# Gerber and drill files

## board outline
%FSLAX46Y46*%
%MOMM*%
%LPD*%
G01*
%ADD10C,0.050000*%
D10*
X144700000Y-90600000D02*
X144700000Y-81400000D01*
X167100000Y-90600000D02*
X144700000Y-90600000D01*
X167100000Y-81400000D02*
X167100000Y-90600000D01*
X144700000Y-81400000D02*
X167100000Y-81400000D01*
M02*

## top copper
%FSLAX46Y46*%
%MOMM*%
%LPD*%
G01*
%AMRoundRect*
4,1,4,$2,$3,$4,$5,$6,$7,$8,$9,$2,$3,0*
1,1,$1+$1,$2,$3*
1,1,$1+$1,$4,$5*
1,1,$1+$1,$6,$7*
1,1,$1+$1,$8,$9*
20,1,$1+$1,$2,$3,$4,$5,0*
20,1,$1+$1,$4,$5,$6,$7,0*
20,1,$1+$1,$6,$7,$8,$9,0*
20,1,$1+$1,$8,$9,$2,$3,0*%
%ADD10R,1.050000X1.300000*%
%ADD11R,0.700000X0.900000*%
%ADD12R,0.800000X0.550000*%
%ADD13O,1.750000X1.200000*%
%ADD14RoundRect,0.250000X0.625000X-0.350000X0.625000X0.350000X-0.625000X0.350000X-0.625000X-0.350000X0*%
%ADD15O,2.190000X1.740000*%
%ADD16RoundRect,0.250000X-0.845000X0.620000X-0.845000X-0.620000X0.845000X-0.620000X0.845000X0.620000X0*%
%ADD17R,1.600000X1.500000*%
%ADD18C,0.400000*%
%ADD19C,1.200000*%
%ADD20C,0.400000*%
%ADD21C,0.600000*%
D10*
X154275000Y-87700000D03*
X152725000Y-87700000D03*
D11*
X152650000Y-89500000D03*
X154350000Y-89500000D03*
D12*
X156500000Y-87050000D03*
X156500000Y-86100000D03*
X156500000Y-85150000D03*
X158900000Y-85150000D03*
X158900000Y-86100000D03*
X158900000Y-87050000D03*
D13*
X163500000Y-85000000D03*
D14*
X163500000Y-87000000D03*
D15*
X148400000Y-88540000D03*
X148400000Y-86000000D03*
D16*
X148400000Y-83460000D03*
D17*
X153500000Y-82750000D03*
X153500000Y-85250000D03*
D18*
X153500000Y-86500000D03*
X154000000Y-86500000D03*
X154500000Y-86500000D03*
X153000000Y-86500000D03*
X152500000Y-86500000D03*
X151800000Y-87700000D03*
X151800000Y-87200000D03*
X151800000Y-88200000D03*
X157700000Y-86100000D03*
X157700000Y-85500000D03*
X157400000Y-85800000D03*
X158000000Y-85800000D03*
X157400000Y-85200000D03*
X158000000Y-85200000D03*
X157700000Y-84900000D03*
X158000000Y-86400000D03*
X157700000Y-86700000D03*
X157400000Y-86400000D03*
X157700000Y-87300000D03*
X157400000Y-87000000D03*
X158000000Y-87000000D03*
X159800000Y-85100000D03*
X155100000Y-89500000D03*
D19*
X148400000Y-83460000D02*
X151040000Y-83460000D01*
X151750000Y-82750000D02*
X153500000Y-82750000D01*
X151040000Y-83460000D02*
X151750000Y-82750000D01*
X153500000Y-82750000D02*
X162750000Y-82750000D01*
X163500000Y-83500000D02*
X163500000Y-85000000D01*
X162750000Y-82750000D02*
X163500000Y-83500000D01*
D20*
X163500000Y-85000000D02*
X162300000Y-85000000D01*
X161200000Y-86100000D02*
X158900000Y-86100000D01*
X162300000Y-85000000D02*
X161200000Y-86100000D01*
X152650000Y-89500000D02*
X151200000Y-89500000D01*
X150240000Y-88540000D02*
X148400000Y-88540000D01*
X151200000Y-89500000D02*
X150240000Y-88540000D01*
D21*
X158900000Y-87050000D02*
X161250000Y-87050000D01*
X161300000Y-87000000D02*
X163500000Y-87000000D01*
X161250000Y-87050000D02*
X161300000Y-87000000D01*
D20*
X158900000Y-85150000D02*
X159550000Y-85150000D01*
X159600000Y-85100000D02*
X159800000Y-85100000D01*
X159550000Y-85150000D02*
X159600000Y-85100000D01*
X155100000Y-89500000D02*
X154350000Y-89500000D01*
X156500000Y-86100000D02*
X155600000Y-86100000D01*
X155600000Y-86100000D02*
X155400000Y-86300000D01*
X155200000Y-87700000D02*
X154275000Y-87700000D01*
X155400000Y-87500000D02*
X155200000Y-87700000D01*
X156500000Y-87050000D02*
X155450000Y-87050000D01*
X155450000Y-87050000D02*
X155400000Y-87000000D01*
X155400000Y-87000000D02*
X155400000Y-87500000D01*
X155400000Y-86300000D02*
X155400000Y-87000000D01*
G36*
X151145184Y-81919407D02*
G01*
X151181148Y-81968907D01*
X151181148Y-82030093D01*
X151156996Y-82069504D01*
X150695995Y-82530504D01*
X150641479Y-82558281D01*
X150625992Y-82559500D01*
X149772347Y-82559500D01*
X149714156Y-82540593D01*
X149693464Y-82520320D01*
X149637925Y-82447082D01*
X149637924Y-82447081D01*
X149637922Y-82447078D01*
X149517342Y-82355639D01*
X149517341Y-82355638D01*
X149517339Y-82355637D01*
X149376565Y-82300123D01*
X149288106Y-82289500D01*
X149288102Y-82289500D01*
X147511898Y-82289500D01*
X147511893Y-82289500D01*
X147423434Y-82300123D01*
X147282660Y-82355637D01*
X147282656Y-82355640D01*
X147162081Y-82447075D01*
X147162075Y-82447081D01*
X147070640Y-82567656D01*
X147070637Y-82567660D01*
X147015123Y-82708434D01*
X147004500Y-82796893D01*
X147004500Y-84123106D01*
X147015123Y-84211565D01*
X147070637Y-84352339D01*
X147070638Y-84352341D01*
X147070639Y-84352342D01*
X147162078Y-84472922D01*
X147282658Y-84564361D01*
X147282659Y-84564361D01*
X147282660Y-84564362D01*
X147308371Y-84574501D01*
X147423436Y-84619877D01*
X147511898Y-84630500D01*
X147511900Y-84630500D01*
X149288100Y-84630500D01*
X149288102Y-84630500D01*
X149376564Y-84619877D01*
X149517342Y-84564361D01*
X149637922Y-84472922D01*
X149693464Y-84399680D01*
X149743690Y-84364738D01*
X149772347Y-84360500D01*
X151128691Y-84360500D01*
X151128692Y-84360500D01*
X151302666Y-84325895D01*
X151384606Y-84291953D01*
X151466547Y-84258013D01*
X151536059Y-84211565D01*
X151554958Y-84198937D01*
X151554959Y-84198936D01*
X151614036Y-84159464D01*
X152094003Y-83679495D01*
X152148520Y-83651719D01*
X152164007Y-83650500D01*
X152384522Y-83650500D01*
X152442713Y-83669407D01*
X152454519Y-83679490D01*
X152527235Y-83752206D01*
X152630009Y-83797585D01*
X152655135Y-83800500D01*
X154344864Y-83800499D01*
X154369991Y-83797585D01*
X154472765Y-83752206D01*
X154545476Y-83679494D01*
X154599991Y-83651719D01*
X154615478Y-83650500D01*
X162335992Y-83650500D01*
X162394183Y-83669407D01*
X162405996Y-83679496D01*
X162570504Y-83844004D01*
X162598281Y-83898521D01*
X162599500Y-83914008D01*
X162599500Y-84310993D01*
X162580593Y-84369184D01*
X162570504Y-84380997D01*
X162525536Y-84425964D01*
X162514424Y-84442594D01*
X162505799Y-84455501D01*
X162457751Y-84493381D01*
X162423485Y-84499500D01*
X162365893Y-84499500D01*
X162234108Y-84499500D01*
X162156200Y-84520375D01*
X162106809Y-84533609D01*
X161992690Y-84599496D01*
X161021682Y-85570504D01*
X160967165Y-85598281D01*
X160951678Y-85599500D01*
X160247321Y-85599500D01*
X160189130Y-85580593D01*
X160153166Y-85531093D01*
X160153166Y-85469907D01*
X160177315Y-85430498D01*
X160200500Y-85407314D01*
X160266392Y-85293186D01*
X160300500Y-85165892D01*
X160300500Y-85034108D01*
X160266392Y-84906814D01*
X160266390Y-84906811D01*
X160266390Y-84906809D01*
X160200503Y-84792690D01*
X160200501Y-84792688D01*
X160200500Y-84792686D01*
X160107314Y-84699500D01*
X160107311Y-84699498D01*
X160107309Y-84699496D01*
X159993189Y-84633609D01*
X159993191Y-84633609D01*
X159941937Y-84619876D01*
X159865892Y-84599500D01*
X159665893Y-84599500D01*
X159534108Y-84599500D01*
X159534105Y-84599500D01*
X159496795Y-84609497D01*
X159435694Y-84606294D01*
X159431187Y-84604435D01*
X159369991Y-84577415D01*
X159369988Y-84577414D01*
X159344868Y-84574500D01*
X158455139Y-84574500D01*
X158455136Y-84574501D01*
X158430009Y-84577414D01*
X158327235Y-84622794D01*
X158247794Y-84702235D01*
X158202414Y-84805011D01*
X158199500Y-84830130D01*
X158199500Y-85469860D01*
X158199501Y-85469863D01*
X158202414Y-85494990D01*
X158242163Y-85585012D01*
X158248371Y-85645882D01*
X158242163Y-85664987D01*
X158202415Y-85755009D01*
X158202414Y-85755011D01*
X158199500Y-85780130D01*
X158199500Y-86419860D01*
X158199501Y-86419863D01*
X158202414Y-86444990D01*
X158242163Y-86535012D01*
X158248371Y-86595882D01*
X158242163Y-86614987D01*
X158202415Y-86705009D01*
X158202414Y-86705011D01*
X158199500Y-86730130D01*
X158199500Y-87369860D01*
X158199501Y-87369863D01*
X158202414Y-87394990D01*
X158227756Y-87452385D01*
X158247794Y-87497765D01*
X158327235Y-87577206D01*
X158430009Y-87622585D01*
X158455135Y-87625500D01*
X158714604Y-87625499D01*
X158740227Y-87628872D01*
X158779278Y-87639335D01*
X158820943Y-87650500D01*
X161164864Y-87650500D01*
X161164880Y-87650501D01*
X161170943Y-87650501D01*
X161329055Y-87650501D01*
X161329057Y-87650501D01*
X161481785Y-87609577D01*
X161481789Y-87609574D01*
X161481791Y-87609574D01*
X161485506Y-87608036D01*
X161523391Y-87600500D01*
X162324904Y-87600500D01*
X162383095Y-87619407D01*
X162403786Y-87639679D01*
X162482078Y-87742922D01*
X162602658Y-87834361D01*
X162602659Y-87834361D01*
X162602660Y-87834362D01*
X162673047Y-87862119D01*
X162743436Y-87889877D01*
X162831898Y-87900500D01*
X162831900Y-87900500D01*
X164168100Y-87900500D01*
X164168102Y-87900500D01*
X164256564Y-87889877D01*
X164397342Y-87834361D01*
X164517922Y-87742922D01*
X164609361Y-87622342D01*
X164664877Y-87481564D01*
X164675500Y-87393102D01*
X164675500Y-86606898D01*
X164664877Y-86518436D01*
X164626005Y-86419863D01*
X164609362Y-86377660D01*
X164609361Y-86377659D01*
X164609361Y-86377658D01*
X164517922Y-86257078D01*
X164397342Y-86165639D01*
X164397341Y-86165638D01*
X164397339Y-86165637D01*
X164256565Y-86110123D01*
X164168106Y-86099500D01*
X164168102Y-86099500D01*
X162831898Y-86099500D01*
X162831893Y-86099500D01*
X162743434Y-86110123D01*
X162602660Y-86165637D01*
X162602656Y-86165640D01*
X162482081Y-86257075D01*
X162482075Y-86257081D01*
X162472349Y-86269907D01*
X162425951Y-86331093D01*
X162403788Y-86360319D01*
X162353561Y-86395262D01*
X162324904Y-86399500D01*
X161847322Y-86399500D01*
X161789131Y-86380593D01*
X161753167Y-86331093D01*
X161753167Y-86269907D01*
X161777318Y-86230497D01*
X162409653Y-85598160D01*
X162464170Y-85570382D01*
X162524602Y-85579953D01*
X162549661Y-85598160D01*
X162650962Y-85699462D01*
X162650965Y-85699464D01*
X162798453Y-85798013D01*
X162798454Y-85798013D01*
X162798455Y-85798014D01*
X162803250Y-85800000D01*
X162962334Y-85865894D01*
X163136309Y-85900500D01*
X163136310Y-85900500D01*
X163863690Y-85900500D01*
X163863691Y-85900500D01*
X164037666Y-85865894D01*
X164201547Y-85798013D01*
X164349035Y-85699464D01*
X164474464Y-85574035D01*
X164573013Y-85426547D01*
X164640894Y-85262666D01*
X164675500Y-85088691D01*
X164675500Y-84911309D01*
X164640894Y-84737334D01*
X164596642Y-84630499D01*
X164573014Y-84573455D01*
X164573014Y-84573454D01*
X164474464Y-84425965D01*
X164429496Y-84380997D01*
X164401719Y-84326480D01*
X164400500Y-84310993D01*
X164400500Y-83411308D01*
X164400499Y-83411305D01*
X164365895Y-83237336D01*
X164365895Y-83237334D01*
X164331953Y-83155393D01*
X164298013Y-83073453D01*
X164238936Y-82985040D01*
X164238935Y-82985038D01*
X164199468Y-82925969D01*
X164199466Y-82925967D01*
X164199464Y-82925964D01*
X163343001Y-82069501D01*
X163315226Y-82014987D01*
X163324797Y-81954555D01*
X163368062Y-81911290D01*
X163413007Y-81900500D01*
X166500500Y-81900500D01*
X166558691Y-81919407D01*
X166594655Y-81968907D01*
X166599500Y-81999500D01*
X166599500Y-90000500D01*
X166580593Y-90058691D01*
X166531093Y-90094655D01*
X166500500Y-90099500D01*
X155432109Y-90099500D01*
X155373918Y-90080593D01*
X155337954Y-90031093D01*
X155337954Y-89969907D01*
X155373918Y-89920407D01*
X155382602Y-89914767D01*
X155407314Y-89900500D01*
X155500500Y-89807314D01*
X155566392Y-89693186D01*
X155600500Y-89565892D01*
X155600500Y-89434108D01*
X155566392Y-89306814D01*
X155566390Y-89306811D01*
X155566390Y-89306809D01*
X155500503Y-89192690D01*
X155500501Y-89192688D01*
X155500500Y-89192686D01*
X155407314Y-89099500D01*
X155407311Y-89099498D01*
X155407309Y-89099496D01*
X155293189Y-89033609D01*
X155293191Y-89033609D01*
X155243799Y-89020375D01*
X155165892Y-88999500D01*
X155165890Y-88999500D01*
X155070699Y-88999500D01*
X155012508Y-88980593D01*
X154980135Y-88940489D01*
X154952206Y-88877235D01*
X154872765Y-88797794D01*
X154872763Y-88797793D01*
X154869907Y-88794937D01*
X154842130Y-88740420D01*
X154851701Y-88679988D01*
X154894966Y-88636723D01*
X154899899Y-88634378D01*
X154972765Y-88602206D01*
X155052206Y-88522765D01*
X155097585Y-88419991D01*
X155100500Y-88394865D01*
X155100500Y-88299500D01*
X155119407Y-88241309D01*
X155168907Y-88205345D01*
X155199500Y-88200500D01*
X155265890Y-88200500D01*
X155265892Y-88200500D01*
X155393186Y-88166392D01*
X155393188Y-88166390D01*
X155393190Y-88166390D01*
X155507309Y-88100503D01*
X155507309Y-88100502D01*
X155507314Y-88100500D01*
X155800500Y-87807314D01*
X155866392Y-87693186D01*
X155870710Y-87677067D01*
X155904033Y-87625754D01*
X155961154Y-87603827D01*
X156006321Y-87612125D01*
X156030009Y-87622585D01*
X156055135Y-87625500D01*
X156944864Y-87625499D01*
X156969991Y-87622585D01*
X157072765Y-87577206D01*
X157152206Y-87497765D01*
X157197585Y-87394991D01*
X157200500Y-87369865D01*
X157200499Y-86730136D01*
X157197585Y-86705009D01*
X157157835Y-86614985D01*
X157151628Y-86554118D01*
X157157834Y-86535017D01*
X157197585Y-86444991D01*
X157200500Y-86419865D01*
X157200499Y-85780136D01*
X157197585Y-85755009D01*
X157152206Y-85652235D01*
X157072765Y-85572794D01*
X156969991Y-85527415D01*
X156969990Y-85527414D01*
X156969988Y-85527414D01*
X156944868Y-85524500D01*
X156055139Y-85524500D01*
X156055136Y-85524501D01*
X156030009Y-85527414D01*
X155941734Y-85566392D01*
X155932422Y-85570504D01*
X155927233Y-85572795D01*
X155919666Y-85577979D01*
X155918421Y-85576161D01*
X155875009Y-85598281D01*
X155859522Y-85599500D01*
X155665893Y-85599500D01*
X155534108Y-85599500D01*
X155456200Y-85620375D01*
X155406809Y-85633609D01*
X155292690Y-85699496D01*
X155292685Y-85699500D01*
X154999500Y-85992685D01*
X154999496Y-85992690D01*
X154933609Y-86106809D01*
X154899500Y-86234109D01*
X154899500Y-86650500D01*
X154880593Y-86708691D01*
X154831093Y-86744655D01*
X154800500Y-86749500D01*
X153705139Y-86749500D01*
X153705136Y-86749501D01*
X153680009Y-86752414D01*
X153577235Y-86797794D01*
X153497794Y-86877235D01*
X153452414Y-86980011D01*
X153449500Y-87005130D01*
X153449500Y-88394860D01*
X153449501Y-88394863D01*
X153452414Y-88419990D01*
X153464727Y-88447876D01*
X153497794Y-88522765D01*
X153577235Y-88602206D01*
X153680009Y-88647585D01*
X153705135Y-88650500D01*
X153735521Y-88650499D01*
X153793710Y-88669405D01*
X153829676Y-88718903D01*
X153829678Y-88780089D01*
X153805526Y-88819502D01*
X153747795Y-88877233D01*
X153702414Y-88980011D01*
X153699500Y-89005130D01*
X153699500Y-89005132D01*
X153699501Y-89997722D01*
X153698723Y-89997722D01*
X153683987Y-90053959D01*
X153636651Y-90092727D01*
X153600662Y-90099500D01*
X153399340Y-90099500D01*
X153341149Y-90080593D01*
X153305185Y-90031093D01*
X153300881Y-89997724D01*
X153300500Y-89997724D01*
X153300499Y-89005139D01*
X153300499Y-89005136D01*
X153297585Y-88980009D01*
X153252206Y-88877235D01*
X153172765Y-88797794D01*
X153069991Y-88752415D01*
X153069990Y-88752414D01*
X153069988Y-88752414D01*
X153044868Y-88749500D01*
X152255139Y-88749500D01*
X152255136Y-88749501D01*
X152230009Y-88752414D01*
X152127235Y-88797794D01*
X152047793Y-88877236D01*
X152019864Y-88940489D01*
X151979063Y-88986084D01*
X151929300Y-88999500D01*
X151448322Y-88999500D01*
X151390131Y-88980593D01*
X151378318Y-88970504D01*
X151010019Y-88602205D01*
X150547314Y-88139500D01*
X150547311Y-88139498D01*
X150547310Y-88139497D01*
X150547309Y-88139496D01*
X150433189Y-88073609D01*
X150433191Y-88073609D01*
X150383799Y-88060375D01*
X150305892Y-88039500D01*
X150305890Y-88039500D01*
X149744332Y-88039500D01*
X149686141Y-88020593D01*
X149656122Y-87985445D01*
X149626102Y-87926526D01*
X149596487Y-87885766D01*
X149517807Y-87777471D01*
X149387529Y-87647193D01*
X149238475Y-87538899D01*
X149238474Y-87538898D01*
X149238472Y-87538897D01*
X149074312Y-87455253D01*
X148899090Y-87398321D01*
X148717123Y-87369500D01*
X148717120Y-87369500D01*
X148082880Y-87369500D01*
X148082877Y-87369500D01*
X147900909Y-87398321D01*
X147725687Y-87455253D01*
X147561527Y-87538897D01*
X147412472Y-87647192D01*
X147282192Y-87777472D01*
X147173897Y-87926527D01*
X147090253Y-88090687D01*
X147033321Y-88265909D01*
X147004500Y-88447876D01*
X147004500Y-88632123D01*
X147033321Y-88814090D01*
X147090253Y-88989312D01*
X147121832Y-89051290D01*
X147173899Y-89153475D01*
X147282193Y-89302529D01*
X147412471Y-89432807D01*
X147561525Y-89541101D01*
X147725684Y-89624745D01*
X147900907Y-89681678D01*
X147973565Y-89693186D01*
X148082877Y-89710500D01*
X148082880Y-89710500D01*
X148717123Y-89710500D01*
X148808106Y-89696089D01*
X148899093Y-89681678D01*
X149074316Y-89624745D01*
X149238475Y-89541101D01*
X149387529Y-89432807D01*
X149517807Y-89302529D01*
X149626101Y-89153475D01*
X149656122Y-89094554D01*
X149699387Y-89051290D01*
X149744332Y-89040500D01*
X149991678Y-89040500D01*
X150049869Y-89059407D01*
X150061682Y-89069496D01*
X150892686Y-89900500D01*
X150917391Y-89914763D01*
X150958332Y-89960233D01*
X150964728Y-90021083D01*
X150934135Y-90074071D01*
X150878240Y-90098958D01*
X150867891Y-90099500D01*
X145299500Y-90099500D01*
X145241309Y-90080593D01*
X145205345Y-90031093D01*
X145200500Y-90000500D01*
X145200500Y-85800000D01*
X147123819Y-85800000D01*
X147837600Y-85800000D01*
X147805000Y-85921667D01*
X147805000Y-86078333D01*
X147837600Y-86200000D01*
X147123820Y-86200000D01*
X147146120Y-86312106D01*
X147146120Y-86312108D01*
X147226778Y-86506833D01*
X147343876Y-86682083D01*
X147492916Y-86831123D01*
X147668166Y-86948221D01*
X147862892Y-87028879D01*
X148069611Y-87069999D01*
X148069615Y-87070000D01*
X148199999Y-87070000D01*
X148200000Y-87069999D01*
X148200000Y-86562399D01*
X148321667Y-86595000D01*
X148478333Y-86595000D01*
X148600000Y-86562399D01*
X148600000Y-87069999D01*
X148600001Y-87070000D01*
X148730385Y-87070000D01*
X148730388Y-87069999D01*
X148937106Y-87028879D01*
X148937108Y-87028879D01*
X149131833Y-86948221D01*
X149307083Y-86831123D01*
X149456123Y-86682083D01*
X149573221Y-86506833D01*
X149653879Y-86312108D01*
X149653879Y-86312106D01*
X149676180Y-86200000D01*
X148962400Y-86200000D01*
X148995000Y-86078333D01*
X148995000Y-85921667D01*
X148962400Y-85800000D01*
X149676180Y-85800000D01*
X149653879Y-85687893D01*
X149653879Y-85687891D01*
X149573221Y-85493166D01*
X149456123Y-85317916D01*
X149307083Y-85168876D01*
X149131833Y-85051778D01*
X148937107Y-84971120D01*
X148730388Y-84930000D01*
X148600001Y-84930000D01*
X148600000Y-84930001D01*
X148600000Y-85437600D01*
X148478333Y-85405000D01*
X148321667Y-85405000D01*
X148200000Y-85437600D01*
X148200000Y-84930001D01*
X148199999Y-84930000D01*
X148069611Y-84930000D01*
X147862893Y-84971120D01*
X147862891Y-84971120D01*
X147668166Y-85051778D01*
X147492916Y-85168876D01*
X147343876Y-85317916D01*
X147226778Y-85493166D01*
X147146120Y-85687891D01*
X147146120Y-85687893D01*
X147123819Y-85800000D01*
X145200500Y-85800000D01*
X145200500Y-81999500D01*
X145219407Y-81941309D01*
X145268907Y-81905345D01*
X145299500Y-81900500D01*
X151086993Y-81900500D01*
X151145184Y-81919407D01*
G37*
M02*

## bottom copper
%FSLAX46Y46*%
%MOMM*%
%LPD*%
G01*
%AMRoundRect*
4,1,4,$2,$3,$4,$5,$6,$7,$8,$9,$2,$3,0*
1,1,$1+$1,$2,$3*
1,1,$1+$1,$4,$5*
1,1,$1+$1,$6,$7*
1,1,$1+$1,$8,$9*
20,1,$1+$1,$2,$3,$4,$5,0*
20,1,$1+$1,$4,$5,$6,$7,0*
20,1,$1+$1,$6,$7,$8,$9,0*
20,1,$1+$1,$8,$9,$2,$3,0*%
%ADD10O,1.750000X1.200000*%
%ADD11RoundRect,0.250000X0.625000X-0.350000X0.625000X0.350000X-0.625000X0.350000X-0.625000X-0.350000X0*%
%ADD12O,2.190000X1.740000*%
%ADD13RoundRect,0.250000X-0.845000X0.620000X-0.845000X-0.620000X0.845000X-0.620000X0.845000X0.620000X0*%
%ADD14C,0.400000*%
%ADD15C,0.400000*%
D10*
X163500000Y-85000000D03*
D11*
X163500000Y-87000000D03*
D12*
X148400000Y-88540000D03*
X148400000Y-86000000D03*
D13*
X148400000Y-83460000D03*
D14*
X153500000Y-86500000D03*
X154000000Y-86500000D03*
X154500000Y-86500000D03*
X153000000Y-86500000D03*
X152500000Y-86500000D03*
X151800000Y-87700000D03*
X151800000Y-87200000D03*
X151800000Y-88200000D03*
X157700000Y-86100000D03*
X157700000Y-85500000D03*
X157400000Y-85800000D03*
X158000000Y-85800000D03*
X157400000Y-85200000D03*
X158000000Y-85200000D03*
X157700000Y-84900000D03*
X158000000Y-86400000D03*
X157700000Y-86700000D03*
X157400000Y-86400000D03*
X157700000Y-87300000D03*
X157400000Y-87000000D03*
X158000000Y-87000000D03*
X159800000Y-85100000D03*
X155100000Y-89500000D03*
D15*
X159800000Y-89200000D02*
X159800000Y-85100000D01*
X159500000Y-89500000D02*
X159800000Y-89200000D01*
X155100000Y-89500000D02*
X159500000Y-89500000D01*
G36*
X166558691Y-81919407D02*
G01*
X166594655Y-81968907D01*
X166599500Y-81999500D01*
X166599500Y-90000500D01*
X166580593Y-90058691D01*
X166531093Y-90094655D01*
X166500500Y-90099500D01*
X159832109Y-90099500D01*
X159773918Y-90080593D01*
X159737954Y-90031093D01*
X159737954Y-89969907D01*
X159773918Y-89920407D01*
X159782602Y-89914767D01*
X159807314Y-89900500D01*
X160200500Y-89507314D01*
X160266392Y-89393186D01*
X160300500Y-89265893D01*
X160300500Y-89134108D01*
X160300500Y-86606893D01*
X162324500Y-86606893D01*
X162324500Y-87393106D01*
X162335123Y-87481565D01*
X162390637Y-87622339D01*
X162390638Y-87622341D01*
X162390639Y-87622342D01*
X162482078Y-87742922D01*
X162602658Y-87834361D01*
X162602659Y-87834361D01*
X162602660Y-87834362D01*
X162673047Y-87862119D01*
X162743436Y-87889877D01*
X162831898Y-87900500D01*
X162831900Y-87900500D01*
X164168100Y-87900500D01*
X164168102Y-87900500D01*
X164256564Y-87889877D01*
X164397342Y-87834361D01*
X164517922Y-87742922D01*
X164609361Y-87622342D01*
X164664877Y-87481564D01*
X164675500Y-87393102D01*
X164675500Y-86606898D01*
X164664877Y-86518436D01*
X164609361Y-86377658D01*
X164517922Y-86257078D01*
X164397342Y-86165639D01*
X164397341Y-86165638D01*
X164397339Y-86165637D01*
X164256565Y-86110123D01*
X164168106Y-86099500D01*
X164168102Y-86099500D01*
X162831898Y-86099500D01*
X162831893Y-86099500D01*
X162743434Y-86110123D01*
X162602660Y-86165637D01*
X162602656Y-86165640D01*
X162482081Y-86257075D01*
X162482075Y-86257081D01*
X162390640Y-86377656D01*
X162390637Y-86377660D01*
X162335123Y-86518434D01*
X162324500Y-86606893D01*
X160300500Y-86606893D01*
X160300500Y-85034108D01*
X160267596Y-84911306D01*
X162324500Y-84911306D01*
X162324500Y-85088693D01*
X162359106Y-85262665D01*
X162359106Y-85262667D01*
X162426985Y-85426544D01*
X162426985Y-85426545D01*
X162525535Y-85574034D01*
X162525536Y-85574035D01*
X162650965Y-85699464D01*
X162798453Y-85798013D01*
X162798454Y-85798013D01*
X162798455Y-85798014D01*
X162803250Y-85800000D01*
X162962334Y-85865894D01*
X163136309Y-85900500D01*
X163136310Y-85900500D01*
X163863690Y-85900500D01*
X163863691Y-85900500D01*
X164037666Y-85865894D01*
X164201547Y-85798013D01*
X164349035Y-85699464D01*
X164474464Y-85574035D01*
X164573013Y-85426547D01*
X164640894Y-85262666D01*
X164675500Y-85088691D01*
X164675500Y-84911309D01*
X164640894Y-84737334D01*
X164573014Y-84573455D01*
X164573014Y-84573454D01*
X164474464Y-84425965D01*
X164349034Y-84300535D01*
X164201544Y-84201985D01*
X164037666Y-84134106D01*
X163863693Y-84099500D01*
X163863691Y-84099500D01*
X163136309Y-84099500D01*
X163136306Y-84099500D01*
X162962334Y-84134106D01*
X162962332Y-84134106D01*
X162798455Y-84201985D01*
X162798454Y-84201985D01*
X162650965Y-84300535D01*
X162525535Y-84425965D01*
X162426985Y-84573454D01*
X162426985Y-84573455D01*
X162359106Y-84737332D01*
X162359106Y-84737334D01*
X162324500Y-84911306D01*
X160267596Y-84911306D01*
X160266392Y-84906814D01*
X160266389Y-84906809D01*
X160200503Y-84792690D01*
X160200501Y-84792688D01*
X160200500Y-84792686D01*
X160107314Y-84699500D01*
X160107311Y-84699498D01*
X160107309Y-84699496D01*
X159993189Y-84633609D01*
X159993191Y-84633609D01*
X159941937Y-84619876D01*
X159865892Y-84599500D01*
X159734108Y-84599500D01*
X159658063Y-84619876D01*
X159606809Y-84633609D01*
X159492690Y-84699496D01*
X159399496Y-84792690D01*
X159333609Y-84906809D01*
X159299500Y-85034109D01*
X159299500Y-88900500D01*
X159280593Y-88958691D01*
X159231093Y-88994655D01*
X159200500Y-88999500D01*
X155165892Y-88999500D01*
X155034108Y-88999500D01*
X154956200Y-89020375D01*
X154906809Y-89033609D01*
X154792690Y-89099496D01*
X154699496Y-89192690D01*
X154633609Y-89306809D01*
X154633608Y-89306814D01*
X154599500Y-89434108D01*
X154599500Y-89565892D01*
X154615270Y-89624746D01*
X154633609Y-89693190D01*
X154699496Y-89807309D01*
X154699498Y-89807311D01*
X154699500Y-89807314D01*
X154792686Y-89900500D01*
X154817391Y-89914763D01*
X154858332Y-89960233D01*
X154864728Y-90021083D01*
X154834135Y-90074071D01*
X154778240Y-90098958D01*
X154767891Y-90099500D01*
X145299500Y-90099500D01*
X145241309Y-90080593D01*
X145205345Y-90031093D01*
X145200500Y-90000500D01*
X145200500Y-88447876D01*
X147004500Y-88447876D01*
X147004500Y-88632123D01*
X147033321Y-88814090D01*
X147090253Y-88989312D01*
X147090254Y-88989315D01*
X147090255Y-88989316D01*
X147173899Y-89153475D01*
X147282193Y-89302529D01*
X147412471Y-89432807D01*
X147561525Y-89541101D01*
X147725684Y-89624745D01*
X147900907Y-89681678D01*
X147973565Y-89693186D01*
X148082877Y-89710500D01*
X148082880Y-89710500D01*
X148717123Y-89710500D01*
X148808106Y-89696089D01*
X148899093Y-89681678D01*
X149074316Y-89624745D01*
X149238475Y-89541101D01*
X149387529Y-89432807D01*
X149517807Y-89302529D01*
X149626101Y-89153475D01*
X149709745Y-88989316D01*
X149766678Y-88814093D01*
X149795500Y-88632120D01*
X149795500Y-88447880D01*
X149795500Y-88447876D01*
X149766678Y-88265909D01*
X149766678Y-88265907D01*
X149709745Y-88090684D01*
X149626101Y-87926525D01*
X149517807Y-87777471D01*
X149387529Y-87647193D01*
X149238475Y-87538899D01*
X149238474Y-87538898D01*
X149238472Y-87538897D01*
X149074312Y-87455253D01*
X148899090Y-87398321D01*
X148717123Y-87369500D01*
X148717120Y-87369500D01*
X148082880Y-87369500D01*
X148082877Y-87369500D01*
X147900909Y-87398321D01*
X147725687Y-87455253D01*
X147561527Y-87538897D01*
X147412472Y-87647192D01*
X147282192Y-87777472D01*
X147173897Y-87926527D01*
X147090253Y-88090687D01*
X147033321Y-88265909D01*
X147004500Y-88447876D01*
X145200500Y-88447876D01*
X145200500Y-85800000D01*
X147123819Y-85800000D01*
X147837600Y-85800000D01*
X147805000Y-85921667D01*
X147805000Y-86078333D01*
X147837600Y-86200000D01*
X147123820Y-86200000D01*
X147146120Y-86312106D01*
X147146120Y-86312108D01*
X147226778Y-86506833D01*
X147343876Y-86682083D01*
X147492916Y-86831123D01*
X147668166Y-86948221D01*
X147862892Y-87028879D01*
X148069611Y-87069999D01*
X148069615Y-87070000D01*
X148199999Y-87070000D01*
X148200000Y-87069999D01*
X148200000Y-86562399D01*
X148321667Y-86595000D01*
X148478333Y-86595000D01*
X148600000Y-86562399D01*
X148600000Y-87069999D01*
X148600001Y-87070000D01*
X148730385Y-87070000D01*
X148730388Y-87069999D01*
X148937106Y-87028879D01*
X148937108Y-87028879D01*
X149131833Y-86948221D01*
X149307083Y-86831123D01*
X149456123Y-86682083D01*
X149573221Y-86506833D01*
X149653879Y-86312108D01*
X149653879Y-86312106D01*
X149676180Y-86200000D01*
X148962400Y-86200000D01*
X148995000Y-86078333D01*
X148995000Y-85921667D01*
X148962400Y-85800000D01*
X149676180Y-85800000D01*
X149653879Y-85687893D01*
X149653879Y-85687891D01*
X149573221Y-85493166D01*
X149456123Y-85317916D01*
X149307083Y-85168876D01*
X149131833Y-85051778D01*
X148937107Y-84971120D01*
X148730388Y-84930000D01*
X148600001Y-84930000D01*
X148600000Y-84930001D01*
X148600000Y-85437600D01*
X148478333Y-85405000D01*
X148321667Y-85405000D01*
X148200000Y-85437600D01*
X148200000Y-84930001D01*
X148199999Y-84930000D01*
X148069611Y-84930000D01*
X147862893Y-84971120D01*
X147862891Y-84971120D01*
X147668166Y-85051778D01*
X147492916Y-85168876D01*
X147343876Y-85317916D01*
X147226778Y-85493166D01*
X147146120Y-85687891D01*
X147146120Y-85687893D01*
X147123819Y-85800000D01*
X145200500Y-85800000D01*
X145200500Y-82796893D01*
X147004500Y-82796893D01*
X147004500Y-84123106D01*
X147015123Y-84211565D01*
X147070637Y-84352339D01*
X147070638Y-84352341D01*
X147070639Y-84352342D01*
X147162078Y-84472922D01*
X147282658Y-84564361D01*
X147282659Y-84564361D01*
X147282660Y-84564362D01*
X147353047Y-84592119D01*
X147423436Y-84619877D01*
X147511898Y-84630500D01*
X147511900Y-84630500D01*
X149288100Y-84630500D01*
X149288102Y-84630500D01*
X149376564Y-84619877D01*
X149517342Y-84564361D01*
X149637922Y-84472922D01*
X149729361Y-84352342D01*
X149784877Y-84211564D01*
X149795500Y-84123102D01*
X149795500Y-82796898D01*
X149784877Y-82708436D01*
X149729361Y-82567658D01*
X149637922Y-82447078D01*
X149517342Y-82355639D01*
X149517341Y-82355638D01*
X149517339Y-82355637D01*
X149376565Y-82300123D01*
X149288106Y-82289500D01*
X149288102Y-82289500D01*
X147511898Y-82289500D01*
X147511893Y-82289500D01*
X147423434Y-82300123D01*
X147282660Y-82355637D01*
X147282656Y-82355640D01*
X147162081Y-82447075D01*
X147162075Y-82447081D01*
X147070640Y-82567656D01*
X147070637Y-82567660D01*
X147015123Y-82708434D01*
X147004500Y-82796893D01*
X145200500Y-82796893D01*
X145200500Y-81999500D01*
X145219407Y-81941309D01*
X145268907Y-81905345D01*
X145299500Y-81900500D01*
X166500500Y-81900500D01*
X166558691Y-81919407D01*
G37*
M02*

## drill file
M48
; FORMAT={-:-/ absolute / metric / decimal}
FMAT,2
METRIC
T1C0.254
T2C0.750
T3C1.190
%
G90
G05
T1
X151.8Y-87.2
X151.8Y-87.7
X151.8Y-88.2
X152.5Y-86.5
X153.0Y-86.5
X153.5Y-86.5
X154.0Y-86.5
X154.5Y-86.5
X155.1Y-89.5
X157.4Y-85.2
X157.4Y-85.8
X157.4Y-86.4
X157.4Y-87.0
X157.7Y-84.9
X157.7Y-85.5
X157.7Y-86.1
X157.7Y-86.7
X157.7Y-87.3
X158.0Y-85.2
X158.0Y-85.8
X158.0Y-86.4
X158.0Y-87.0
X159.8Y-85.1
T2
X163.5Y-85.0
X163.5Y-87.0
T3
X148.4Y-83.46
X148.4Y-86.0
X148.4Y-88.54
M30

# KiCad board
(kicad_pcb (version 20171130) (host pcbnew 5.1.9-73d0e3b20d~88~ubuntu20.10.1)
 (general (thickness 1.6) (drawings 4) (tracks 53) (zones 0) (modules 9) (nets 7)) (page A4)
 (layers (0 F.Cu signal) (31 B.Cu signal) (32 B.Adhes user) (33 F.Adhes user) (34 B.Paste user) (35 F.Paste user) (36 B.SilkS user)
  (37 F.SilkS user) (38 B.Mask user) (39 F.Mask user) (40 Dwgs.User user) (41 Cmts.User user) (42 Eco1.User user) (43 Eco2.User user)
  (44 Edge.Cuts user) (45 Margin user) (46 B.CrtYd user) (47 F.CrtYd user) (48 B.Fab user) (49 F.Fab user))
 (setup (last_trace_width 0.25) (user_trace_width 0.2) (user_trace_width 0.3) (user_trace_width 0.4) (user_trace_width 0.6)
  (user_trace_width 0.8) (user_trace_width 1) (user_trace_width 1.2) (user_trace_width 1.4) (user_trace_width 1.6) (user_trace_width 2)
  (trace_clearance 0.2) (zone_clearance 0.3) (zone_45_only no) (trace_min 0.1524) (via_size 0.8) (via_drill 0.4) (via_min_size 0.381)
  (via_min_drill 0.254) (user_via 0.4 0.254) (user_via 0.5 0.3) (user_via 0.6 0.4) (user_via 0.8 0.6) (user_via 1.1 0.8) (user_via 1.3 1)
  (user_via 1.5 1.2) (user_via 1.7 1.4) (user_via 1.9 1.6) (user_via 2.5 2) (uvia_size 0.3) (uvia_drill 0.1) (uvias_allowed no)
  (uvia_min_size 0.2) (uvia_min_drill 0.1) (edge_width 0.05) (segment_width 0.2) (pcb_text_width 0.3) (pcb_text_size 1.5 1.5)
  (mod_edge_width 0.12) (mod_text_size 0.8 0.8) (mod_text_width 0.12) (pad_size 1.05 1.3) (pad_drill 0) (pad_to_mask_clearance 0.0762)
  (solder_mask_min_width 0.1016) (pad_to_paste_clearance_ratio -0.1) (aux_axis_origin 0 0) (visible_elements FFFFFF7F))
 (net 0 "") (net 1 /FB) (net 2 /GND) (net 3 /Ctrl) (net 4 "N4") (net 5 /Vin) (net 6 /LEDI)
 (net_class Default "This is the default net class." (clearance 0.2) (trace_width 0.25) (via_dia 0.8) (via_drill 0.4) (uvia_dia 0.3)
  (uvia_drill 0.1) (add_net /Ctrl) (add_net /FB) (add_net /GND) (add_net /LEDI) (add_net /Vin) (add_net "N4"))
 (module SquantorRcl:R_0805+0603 (layer F.Cu) (at 153.5 87.7)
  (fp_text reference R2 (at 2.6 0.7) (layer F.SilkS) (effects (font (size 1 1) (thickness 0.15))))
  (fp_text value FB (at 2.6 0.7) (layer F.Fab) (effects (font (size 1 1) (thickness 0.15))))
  (pad 2 smd rect (at 0.775 0) (size 1.05 1.3) (layers F.Cu F.Paste F.Mask) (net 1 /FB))
  (pad 1 smd rect (at -0.775 0) (size 1.05 1.3) (layers F.Cu F.Paste F.Mask) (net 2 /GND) (zone_connect 2)))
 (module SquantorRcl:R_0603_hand (layer F.Cu) (at 153.5 89.5 180)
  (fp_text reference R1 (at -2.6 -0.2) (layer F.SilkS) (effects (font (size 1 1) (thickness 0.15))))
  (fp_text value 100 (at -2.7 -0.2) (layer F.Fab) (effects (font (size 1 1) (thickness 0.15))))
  (pad 2 smd rect (at 0.85 0 180) (size 0.7 0.9) (layers F.Cu F.Paste F.Mask) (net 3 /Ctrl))
  (pad 1 smd rect (at -0.85 0 180) (size 0.7 0.9) (layers F.Cu F.Paste F.Mask) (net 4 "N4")))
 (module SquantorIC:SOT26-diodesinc (layer F.Cu) (at 157.7 86.1 90)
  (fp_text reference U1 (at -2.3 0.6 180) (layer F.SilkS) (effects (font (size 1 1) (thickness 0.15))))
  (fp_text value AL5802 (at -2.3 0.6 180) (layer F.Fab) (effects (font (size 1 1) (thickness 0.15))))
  (pad 6 smd rect (at -0.95 -1.2 90) (size 0.55 0.8) (layers F.Cu F.Paste F.Mask) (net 1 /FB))
  (pad 5 smd rect (at 0 -1.2 90) (size 0.55 0.8) (layers F.Cu F.Paste F.Mask) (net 1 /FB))
  (pad 4 smd rect (at 0.95 -1.2 90) (size 0.55 0.8) (layers F.Cu F.Paste F.Mask) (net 2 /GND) (zone_connect 2))
  (pad 3 smd rect (at 0.95 1.2 90) (size 0.55 0.8) (layers F.Cu F.Paste F.Mask) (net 4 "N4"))
  (pad 2 smd rect (at 0 1.2 90) (size 0.55 0.8) (layers F.Cu F.Paste F.Mask) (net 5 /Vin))
  (pad 1 smd rect (at -0.95 1.2 90) (size 0.55 0.8) (layers F.Cu F.Paste F.Mask) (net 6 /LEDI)))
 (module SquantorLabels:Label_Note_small (layer F.Cu) (at 156 82.9)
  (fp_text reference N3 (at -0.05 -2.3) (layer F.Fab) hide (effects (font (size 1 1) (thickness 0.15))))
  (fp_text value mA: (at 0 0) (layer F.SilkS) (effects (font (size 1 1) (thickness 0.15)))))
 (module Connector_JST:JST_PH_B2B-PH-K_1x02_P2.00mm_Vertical (layer F.Cu) (at 163.5 87 90)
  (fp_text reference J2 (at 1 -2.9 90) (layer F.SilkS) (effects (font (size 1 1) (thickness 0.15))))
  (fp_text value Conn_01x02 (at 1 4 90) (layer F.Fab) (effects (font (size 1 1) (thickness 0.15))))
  (pad 2 thru_hole oval (at 2 0 90) (size 1.2 1.75) (drill 0.75) (layers *.Cu *.Mask) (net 5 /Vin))
  (pad 1 thru_hole roundrect (at 0 0 90) (size 1.2 1.75) (drill 0.75) (layers *.Cu *.Mask) (roundrect_rratio 0.208333) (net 6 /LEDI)))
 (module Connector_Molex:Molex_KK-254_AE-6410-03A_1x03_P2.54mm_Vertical (layer F.Cu) (at 148.4 83.46 270)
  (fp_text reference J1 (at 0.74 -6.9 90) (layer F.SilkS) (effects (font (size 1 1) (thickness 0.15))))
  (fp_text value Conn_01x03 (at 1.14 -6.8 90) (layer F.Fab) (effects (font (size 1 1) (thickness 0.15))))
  (pad 3 thru_hole oval (at 5.08 0 270) (size 1.74 2.19) (drill 1.19) (layers *.Cu *.Mask) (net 3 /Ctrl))
  (pad 2 thru_hole oval (at 2.54 0 270) (size 1.74 2.19) (drill 1.19) (layers *.Cu *.Mask) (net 2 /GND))
  (pad 1 thru_hole roundrect (at 0 0 270) (size 1.74 2.19) (drill 1.19) (layers *.Cu *.Mask) (roundrect_rratio 0.143678) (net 5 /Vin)))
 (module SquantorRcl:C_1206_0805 (layer F.Cu) (at 153.5 84 90)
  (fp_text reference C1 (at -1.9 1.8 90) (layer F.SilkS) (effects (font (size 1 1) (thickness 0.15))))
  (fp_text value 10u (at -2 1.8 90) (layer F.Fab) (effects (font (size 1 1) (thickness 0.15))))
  (pad 2 smd rect (at 1.25 0 90) (size 1.5 1.6) (layers F.Cu F.Paste F.Mask) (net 5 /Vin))
  (pad 1 smd rect (at -1.25 0 90) (size 1.5 1.6) (layers F.Cu F.Paste F.Mask) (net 2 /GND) (zone_connect 2)))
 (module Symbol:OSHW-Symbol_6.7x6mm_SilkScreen (layer B.Cu) (at 155.5 86 270)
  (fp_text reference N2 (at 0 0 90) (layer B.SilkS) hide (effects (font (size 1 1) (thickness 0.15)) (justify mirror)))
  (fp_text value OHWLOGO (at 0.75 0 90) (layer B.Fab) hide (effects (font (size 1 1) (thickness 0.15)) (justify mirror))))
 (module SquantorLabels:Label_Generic (layer B.Cu) (at 159.2 85.2 270)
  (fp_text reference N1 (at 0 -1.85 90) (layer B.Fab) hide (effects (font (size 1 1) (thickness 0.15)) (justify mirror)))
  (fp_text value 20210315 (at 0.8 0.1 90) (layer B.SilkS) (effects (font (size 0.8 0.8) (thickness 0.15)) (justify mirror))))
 (gr_line (start 144.7 90.6) (end 144.7 81.4) (layer Edge.Cuts) (width 0.05))
 (gr_line (start 167.1 90.6) (end 144.7 90.6) (layer Edge.Cuts) (width 0.05))
 (gr_line (start 167.1 81.4) (end 167.1 90.6) (layer Edge.Cuts) (width 0.05))
 (gr_line (start 144.7 81.4) (end 167.1 81.4) (layer Edge.Cuts) (width 0.05))
 (segment (start 148.4 83.46) (end 151.04 83.46) (width 1.2) (layer F.Cu) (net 5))
 (segment (start 151.75 82.75) (end 153.5 82.75) (width 1.2) (layer F.Cu) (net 5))
 (segment (start 151.04 83.46) (end 151.75 82.75) (width 1.2) (layer F.Cu) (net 5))
 (segment (start 153.5 82.75) (end 162.75 82.75) (width 1.2) (layer F.Cu) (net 5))
 (segment (start 163.5 83.5) (end 163.5 85) (width 1.2) (layer F.Cu) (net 5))
 (segment (start 162.75 82.75) (end 163.5 83.5) (width 1.2) (layer F.Cu) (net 5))
 (segment (start 163.5 85) (end 162.3 85) (width 0.4) (layer F.Cu) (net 5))
 (segment (start 161.2 86.1) (end 158.9 86.1) (width 0.4) (layer F.Cu) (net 5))
 (segment (start 162.3 85) (end 161.2 86.1) (width 0.4) (layer F.Cu) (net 5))
 (via (at 153.5 86.5) (size 0.4) (drill 0.254) (layers F.Cu B.Cu) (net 2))
 (via (at 154 86.5) (size 0.4) (drill 0.254) (layers F.Cu B.Cu) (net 2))
 (via (at 154.5 86.5) (size 0.4) (drill 0.254) (layers F.Cu B.Cu) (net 2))
 (via (at 153 86.5) (size 0.4) (drill 0.254) (layers F.Cu B.Cu) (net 2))
 (via (at 152.5 86.5) (size 0.4) (drill 0.254) (layers F.Cu B.Cu) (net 2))
 (via (at 151.8 87.7) (size 0.4) (drill 0.254) (layers F.Cu B.Cu) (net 2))
 (via (at 151.8 87.2) (size 0.4) (drill 0.254) (layers F.Cu B.Cu) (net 2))
 (via (at 151.8 88.2) (size 0.4) (drill 0.254) (layers F.Cu B.Cu) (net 2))
 (via (at 157.7 86.1) (size 0.4) (drill 0.254) (layers F.Cu B.Cu) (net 2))
 (via (at 157.7 85.5) (size 0.4) (drill 0.254) (layers F.Cu B.Cu) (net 2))
 (via (at 157.4 85.8) (size 0.4) (drill 0.254) (layers F.Cu B.Cu) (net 2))
 (via (at 158 85.8) (size 0.4) (drill 0.254) (layers F.Cu B.Cu) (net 2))
 (via (at 157.4 85.2) (size 0.4) (drill 0.254) (layers F.Cu B.Cu) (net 2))
 (via (at 158 85.2) (size 0.4) (drill 0.254) (layers F.Cu B.Cu) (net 2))
 (via (at 157.7 84.9) (size 0.4) (drill 0.254) (layers F.Cu B.Cu) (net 2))
 (via (at 158 86.4) (size 0.4) (drill 0.254) (layers F.Cu B.Cu) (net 2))
 (via (at 157.7 86.7) (size 0.4) (drill 0.254) (layers F.Cu B.Cu) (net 2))
 (via (at 157.4 86.4) (size 0.4) (drill 0.254) (layers F.Cu B.Cu) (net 2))
 (via (at 157.7 87.3) (size 0.4) (drill 0.254) (layers F.Cu B.Cu) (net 2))
 (via (at 157.4 87) (size 0.4) (drill 0.254) (layers F.Cu B.Cu) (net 2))
 (via (at 158 87) (size 0.4) (drill 0.254) (layers F.Cu B.Cu) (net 2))
 (segment (start 152.65 89.5) (end 151.2 89.5) (width 0.4) (layer F.Cu) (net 3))
 (segment (start 150.24 88.54) (end 148.4 88.54) (width 0.4) (layer F.Cu) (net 3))
 (segment (start 151.2 89.5) (end 150.24 88.54) (width 0.4) (layer F.Cu) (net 3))
 (segment (start 158.9 87.05) (end 161.25 87.05) (width 0.6) (layer F.Cu) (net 6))
 (segment (start 161.3 87) (end 163.5 87) (width 0.6) (layer F.Cu) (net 6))
 (segment (start 161.25 87.05) (end 161.3 87) (width 0.6) (layer F.Cu) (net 6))
 (segment (start 158.9 85.15) (end 159.55 85.15) (width 0.4) (layer F.Cu) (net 4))
 (via (at 159.8 85.1) (size 0.4) (drill 0.254) (layers F.Cu B.Cu) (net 4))
 (segment (start 159.6 85.1) (end 159.8 85.1) (width 0.4) (layer F.Cu) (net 4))
 (segment (start 159.55 85.15) (end 159.6 85.1) (width 0.4) (layer F.Cu) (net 4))
 (segment (start 155.1 89.5) (end 154.35 89.5) (width 0.4) (layer F.Cu) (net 4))
 (segment (start 159.8 89.2) (end 159.8 85.1) (width 0.4) (layer B.Cu) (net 4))
 (segment (start 159.5 89.5) (end 159.8 89.2) (width 0.4) (layer B.Cu) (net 4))
 (segment (start 155.1 89.5) (end 159.5 89.5) (width 0.4) (layer B.Cu) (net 4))
 (via (at 155.1 89.5) (size 0.4) (drill 0.254) (layers F.Cu B.Cu) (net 4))
 (segment (start 156.5 86.1) (end 155.6 86.1) (width 0.4) (layer F.Cu) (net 1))
 (segment (start 155.6 86.1) (end 155.4 86.3) (width 0.4) (layer F.Cu) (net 1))
 (segment (start 155.2 87.7) (end 154.275 87.7) (width 0.4) (layer F.Cu) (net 1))
 (segment (start 155.4 87.5) (end 155.2 87.7) (width 0.4) (layer F.Cu) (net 1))
 (segment (start 156.5 87.05) (end 155.45 87.05) (width 0.4) (layer F.Cu) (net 1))
 (segment (start 155.45 87.05) (end 155.4 87) (width 0.4) (layer F.Cu) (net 1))
 (segment (start 155.4 87) (end 155.4 87.5) (width 0.4) (layer F.Cu) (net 1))
 (segment (start 155.4 86.3) (end 155.4 87) (width 0.4) (layer F.Cu) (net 1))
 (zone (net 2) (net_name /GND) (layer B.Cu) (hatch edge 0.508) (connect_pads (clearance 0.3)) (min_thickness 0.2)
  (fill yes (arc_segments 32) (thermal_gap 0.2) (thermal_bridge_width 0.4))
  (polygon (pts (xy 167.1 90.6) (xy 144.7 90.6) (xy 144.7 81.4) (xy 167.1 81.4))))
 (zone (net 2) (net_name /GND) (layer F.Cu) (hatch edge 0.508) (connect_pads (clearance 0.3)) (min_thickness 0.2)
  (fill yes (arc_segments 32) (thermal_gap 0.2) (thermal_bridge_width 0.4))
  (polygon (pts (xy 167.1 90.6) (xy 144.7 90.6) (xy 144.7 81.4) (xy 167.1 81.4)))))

